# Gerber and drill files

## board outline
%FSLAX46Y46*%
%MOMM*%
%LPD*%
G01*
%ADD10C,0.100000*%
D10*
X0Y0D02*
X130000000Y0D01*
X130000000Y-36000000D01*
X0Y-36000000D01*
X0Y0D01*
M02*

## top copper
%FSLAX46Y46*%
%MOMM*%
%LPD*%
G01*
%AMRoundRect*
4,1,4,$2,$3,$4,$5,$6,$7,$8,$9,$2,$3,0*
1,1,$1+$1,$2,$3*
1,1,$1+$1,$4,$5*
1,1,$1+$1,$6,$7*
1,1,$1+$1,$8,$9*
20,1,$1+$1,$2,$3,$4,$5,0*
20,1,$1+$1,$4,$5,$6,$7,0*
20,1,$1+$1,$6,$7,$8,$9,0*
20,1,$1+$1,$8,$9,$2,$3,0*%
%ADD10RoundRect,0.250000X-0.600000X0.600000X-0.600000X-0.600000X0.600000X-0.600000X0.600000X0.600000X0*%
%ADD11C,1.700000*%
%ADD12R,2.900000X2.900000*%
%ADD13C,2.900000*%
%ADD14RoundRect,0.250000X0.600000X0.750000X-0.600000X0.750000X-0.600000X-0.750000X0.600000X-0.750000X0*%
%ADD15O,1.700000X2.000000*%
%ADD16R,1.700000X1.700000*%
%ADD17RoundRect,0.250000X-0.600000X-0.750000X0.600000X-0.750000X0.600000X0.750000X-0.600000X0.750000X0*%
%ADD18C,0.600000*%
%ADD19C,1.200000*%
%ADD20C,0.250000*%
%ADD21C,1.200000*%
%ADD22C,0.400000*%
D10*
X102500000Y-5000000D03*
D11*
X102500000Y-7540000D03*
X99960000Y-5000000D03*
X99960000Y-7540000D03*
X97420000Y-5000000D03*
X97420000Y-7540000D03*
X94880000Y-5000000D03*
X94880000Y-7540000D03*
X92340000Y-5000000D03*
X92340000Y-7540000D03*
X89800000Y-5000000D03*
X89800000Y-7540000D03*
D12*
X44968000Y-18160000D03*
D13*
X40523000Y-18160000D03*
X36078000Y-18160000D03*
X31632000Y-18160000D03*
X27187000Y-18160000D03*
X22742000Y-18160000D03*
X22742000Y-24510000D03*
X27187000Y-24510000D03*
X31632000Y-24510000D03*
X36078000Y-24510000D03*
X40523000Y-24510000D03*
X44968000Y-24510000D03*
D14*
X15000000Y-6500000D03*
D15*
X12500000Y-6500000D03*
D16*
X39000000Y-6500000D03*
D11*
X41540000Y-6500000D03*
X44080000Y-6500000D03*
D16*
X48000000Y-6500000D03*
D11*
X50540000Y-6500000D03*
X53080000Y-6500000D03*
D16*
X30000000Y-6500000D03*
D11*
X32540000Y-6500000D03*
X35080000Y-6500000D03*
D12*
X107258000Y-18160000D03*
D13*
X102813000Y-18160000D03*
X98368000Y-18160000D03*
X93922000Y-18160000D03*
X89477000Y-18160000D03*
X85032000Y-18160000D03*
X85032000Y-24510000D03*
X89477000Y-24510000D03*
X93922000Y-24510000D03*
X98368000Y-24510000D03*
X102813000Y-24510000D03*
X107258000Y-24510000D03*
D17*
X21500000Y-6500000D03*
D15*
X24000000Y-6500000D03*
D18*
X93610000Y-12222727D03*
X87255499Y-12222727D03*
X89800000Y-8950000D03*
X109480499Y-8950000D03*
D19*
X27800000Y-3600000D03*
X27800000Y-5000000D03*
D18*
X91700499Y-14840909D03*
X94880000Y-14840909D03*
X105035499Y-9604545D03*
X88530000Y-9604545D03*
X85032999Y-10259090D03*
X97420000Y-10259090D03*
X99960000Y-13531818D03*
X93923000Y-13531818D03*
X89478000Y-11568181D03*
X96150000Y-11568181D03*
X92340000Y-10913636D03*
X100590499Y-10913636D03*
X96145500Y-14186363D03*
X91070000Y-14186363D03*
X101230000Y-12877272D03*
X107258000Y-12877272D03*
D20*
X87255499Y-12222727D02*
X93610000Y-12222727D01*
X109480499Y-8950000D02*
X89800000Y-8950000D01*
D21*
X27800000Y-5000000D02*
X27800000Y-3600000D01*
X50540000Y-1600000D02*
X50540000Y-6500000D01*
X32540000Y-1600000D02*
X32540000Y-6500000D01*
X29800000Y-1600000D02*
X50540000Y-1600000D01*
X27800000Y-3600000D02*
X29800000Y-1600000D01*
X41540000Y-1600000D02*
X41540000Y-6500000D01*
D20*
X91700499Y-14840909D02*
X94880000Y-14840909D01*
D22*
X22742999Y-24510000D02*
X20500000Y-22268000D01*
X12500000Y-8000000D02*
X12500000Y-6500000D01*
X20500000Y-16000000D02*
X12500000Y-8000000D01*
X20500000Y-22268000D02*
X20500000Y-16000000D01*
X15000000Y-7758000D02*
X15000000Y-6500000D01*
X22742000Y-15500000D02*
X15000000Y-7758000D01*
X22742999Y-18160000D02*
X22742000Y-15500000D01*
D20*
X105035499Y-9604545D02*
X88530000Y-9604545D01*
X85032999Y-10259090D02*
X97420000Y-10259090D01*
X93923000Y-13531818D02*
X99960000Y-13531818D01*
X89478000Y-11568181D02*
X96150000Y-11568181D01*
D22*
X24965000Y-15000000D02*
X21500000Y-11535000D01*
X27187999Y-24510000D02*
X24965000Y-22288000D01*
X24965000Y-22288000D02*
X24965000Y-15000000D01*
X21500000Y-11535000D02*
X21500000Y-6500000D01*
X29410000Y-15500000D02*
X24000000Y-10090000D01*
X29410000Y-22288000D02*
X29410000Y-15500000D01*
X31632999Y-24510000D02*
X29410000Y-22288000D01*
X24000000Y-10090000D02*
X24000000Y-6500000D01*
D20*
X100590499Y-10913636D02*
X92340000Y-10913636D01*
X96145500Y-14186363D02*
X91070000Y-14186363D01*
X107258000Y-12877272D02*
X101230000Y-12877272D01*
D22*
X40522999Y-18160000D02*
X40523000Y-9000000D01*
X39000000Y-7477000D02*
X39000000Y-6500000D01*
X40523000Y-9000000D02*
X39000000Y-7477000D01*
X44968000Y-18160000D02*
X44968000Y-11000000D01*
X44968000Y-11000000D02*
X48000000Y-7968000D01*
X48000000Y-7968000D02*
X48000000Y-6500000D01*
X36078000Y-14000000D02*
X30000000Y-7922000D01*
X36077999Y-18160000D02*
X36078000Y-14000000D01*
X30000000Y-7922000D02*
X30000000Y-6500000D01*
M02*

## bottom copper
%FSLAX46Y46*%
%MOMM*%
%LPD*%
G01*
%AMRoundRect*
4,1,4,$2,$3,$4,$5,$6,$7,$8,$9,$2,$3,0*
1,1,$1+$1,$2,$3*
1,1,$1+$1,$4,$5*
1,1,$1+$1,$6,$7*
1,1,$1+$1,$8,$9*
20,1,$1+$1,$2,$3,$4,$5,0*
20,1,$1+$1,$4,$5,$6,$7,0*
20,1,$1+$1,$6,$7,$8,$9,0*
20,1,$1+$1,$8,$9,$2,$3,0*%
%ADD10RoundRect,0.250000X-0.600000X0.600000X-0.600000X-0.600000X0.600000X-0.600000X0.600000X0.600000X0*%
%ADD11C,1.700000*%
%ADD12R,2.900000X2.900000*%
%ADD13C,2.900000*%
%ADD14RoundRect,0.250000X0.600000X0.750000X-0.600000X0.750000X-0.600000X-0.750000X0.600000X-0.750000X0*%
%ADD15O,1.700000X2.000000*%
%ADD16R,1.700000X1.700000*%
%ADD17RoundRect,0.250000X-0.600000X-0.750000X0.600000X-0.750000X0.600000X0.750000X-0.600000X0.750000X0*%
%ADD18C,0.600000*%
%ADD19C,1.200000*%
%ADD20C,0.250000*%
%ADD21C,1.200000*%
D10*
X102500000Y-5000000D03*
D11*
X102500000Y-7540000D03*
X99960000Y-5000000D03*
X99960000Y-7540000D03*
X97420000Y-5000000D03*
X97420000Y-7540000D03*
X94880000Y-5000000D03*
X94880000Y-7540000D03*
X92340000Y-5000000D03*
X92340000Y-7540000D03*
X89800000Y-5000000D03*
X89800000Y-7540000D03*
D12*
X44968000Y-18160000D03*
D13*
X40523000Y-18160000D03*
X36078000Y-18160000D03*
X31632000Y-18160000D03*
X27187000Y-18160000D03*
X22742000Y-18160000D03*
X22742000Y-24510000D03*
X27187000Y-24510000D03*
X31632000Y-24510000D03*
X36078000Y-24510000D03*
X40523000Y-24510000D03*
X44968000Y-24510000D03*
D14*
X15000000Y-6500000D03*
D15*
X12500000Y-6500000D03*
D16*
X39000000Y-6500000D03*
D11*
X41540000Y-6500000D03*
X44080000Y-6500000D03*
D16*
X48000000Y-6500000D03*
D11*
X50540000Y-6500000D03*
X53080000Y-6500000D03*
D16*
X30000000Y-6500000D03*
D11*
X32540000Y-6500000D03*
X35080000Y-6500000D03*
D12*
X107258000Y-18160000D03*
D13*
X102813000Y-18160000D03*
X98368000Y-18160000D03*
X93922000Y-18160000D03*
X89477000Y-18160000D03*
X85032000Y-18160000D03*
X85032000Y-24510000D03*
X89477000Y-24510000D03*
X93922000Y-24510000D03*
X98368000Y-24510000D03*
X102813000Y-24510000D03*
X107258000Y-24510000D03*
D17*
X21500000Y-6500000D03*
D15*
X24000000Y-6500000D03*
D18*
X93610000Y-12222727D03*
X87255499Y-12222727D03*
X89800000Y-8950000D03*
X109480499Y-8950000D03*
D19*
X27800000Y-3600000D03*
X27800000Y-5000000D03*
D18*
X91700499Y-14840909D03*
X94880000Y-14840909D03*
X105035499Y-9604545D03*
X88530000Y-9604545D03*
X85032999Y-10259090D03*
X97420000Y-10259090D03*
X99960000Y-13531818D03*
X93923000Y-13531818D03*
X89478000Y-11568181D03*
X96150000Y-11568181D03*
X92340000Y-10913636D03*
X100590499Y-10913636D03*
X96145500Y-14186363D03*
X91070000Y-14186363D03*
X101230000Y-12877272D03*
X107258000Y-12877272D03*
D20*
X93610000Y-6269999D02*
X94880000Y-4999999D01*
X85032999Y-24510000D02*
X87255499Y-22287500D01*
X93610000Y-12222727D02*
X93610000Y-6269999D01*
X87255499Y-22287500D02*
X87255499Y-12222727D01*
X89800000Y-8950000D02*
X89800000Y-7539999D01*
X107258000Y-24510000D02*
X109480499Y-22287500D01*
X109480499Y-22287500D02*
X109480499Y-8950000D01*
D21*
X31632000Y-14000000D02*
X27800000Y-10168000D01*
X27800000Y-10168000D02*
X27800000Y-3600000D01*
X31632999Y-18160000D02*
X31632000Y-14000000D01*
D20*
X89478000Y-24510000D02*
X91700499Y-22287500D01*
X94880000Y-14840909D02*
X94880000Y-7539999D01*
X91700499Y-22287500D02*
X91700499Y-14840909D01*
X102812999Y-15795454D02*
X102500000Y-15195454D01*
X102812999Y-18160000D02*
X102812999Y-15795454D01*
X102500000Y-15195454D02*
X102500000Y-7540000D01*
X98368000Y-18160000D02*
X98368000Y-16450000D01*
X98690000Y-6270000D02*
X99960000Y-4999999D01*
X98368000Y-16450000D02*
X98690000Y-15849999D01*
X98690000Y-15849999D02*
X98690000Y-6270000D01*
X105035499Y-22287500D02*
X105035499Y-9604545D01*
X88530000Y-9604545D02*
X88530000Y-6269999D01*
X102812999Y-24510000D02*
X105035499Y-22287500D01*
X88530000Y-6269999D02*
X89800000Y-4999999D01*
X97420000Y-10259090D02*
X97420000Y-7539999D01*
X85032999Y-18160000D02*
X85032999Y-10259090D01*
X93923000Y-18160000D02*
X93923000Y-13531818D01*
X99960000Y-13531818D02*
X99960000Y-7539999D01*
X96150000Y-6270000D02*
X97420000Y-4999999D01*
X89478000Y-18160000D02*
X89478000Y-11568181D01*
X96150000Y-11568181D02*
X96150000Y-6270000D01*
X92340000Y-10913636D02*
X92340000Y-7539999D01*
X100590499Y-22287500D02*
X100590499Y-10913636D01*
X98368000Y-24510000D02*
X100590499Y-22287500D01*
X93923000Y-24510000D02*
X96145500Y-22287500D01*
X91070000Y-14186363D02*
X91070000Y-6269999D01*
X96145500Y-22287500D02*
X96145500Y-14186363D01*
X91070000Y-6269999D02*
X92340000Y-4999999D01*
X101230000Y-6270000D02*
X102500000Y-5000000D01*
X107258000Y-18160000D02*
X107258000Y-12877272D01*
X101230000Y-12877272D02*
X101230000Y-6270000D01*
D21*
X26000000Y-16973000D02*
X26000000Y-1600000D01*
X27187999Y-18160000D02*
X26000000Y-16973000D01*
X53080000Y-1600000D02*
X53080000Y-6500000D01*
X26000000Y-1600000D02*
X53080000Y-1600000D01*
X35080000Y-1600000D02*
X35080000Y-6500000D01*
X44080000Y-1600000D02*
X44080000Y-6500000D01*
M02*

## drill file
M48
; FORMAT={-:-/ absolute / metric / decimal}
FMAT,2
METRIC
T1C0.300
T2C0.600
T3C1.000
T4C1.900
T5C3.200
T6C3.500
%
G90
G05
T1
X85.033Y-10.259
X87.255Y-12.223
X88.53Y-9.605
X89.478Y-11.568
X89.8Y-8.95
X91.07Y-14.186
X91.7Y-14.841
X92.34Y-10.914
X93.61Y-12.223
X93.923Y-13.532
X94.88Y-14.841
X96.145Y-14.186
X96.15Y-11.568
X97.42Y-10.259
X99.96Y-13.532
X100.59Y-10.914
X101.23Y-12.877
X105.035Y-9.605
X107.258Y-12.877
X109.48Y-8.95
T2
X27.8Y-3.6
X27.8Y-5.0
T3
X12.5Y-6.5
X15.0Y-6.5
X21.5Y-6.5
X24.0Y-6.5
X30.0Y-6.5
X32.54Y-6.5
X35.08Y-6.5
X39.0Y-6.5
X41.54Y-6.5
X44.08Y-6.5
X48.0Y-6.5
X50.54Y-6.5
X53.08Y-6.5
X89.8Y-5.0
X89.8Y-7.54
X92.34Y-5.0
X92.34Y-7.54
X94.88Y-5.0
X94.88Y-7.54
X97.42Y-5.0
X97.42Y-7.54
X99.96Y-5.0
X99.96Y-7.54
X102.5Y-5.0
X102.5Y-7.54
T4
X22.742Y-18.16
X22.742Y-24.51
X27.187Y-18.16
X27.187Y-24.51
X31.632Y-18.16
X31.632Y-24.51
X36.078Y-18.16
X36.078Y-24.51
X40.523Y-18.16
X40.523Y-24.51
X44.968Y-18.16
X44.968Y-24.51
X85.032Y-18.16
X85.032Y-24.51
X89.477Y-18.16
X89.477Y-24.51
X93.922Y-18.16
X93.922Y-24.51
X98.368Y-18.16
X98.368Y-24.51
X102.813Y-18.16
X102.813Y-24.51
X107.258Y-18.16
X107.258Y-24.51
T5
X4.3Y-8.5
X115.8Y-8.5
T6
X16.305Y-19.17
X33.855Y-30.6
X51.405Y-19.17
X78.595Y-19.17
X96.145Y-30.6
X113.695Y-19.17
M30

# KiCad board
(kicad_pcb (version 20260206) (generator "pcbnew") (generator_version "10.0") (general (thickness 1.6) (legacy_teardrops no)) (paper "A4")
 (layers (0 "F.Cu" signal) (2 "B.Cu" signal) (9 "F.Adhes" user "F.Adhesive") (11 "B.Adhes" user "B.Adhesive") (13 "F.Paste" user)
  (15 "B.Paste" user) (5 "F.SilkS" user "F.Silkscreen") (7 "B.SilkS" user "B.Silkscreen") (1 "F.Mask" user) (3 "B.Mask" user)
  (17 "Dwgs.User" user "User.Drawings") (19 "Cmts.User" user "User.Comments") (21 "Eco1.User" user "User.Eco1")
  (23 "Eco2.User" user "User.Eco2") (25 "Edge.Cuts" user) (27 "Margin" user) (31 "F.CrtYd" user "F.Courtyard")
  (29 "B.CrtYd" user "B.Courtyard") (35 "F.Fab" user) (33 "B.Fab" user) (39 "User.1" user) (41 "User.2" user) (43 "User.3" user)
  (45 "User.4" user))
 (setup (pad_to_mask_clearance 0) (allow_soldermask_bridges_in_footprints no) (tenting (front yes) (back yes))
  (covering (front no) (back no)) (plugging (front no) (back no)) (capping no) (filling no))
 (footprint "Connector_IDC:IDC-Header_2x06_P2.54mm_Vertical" (layer "F.Cu") (at 102.5 5 -90)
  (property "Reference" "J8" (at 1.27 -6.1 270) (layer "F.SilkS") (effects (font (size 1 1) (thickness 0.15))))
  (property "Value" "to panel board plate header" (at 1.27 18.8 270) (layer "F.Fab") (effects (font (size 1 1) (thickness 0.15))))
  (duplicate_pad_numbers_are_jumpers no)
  (pad "1" thru_hole roundrect (at 0 0 270) (size 1.7 1.7) (drill 1) (layers "*.Cu" "*.Mask") (remove_unused_layers no)
   (roundrect_rratio 0.147059) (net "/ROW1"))
  (pad "2" thru_hole circle (at 2.54 0 270) (size 1.7 1.7) (drill 1) (layers "*.Cu" "*.Mask") (remove_unused_layers no) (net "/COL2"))
  (pad "3" thru_hole circle (at 0 2.54 270) (size 1.7 1.7) (drill 1) (layers "*.Cu" "*.Mask") (remove_unused_layers no) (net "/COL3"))
  (pad "4" thru_hole circle (at 2.54 2.54 270) (size 1.7 1.7) (drill 1) (layers "*.Cu" "*.Mask") (remove_unused_layers no) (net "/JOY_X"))
  (pad "5" thru_hole circle (at 0 5.08 270) (size 1.7 1.7) (drill 1) (layers "*.Cu" "*.Mask") (remove_unused_layers no) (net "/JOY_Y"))
  (pad "6" thru_hole circle (at 2.54 5.08 270) (size 1.7 1.7) (drill 1) (layers "*.Cu" "*.Mask") (remove_unused_layers no)
   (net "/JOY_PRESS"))
  (pad "7" thru_hole circle (at 0 7.62 270) (size 1.7 1.7) (drill 1) (layers "*.Cu" "*.Mask") (remove_unused_layers no) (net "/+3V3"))
  (pad "8" thru_hole circle (at 2.54 7.62 270) (size 1.7 1.7) (drill 1) (layers "*.Cu" "*.Mask") (remove_unused_layers no) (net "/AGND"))
  (pad "9" thru_hole circle (at 0 10.16 270) (size 1.7 1.7) (drill 1) (layers "*.Cu" "*.Mask") (remove_unused_layers no) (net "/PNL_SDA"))
  (pad "10" thru_hole circle (at 2.54 10.16 270) (size 1.7 1.7) (drill 1) (layers "*.Cu" "*.Mask") (remove_unused_layers no)
   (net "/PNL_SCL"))
  (pad "11" thru_hole circle (at 0 12.7 270) (size 1.7 1.7) (drill 1) (layers "*.Cu" "*.Mask") (remove_unused_layers no) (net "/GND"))
  (pad "12" thru_hole circle (at 2.54 12.7 270) (size 1.7 1.7) (drill 1) (layers "*.Cu" "*.Mask") (remove_unused_layers no) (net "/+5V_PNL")))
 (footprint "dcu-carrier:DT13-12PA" (layer "F.Cu") (at 33.855 19.17)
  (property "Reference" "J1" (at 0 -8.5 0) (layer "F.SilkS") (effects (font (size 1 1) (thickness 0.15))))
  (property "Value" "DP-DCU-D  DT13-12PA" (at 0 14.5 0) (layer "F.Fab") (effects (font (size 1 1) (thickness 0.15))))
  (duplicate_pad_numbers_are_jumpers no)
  (pad "" np_thru_hole circle (at -17.55 0) (size 3.5 3.5) (drill 3.5) (layers "*.Cu" "*.Mask"))
  (pad "" np_thru_hole circle (at 0 11.43) (size 3.5 3.5) (drill 3.5) (layers "*.Cu" "*.Mask"))
  (pad "" np_thru_hole circle (at 17.55 0) (size 3.5 3.5) (drill 3.5) (layers "*.Cu" "*.Mask"))
  (pad "1" thru_hole rect (at 11.113 -1.01) (size 2.9 2.9) (drill 1.9) (layers "*.Cu" "*.Mask") (remove_unused_layers no) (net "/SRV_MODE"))
  (pad "2" thru_hole circle (at 6.668 -1.01) (size 2.9 2.9) (drill 1.9) (layers "*.Cu" "*.Mask") (remove_unused_layers no)
   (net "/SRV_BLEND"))
  (pad "3" thru_hole circle (at 2.223 -1.01) (size 2.9 2.9) (drill 1.9) (layers "*.Cu" "*.Mask") (remove_unused_layers no)
   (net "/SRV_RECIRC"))
  (pad "4" thru_hole circle (at -2.223 -1.01) (size 2.9 2.9) (drill 1.9) (layers "*.Cu" "*.Mask") (remove_unused_layers no)
   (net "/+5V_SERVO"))
  (pad "5" thru_hole circle (at -6.668 -1.01) (size 2.9 2.9) (drill 1.9) (layers "*.Cu" "*.Mask") (remove_unused_layers no)
   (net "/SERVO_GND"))
  (pad "6" thru_hole circle (at -11.113 -1.01) (size 2.9 2.9) (drill 1.9) (layers "*.Cu" "*.Mask") (remove_unused_layers no)
   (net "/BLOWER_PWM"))
  (pad "7" thru_hole circle (at -11.113 5.34) (size 2.9 2.9) (drill 1.9) (layers "*.Cu" "*.Mask") (remove_unused_layers no)
   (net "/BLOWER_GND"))
  (pad "8" thru_hole circle (at -6.668 5.34) (size 2.9 2.9) (drill 1.9) (layers "*.Cu" "*.Mask") (remove_unused_layers no)
   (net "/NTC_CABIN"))
  (pad "9" thru_hole circle (at -2.223 5.34) (size 2.9 2.9) (drill 1.9) (layers "*.Cu" "*.Mask") (remove_unused_layers no) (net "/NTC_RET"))
  (pad "10" thru_hole circle (at 2.223 5.34) (size 2.9 2.9) (drill 1.9) (layers "*.Cu" "*.Mask") (remove_unused_layers no)
   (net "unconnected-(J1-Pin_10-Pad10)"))
  (pad "11" thru_hole circle (at 6.668 5.34) (size 2.9 2.9) (drill 1.9) (layers "*.Cu" "*.Mask") (remove_unused_layers no)
   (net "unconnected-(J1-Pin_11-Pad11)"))
  (pad "12" thru_hole circle (at 11.113 5.34) (size 2.9 2.9) (drill 1.9) (layers "*.Cu" "*.Mask") (remove_unused_layers no)
   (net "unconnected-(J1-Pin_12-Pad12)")))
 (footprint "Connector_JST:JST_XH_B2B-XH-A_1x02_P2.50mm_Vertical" (layer "F.Cu") (at 15 6.5 180)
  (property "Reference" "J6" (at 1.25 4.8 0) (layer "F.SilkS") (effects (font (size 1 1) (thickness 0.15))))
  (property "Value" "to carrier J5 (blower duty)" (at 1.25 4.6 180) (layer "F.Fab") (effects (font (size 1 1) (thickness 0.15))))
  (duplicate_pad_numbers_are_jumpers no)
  (pad "1" thru_hole roundrect (at 0 0 180) (size 1.7 2) (drill 1) (layers "*.Cu" "*.Mask") (remove_unused_layers no)
   (roundrect_rratio 0.147059) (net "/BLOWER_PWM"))
  (pad "2" thru_hole oval (at 2.5 0 180) (size 1.7 2) (drill 1) (layers "*.Cu" "*.Mask") (remove_unused_layers no) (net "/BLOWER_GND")))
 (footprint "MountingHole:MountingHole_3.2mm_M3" (layer "F.Cu") (at 115.8 8.5)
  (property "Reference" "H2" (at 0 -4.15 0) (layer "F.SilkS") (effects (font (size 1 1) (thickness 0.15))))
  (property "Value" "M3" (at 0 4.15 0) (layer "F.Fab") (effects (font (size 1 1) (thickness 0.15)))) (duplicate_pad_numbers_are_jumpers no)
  (pad "" np_thru_hole circle (at 0 0) (size 3.2 3.2) (drill 3.2) (layers "*.Cu" "*.Mask")))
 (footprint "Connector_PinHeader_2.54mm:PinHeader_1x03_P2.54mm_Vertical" (layer "F.Cu") (at 39 6.5 90)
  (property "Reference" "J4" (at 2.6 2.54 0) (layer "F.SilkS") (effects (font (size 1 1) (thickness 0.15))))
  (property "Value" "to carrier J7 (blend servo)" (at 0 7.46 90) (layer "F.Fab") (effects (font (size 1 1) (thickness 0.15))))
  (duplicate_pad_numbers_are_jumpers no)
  (pad "1" thru_hole rect (at 0 0 90) (size 1.7 1.7) (drill 1) (layers "*.Cu" "*.Mask") (remove_unused_layers no) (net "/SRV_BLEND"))
  (pad "2" thru_hole circle (at 0 2.54 90) (size 1.7 1.7) (drill 1) (layers "*.Cu" "*.Mask") (remove_unused_layers no) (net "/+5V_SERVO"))
  (pad "3" thru_hole circle (at 0 5.08 90) (size 1.7 1.7) (drill 1) (layers "*.Cu" "*.Mask") (remove_unused_layers no) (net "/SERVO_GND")))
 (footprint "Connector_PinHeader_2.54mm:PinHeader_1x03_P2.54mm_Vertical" (layer "F.Cu") (at 48 6.5 90)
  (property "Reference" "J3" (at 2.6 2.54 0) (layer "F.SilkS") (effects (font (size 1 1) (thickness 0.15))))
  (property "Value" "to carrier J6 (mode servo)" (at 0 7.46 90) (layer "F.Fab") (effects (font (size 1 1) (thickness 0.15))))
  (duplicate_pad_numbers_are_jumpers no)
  (pad "1" thru_hole rect (at 0 0 90) (size 1.7 1.7) (drill 1) (layers "*.Cu" "*.Mask") (remove_unused_layers no) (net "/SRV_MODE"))
  (pad "2" thru_hole circle (at 0 2.54 90) (size 1.7 1.7) (drill 1) (layers "*.Cu" "*.Mask") (remove_unused_layers no) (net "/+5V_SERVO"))
  (pad "3" thru_hole circle (at 0 5.08 90) (size 1.7 1.7) (drill 1) (layers "*.Cu" "*.Mask") (remove_unused_layers no) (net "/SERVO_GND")))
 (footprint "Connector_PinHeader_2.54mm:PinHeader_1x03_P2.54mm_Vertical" (layer "F.Cu") (at 30 6.5 90)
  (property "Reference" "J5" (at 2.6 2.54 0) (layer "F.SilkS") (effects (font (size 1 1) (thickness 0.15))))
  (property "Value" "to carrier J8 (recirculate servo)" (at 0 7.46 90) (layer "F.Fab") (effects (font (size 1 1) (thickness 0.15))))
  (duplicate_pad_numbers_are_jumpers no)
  (pad "1" thru_hole rect (at 0 0 90) (size 1.7 1.7) (drill 1) (layers "*.Cu" "*.Mask") (remove_unused_layers no) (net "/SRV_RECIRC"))
  (pad "2" thru_hole circle (at 0 2.54 90) (size 1.7 1.7) (drill 1) (layers "*.Cu" "*.Mask") (remove_unused_layers no) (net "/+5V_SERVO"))
  (pad "3" thru_hole circle (at 0 5.08 90) (size 1.7 1.7) (drill 1) (layers "*.Cu" "*.Mask") (remove_unused_layers no) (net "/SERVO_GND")))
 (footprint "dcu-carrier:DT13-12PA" (layer "F.Cu") (at 96.145 19.17)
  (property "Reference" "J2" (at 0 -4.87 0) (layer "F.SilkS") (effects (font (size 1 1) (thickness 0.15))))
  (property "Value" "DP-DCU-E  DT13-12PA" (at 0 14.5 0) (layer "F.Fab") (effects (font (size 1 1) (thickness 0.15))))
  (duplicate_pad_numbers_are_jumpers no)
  (pad "" np_thru_hole circle (at -17.55 0) (size 3.5 3.5) (drill 3.5) (layers "*.Cu" "*.Mask"))
  (pad "" np_thru_hole circle (at 0 11.43) (size 3.5 3.5) (drill 3.5) (layers "*.Cu" "*.Mask"))
  (pad "" np_thru_hole circle (at 17.55 0) (size 3.5 3.5) (drill 3.5) (layers "*.Cu" "*.Mask"))
  (pad "1" thru_hole rect (at 11.113 -1.01) (size 2.9 2.9) (drill 1.9) (layers "*.Cu" "*.Mask") (remove_unused_layers no) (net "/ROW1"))
  (pad "2" thru_hole circle (at 6.668 -1.01) (size 2.9 2.9) (drill 1.9) (layers "*.Cu" "*.Mask") (remove_unused_layers no) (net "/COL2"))
  (pad "3" thru_hole circle (at 2.223 -1.01) (size 2.9 2.9) (drill 1.9) (layers "*.Cu" "*.Mask") (remove_unused_layers no) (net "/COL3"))
  (pad "4" thru_hole circle (at -2.223 -1.01) (size 2.9 2.9) (drill 1.9) (layers "*.Cu" "*.Mask") (remove_unused_layers no) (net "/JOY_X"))
  (pad "5" thru_hole circle (at -6.668 -1.01) (size 2.9 2.9) (drill 1.9) (layers "*.Cu" "*.Mask") (remove_unused_layers no) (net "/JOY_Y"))
  (pad "6" thru_hole circle (at -11.113 -1.01) (size 2.9 2.9) (drill 1.9) (layers "*.Cu" "*.Mask") (remove_unused_layers no)
   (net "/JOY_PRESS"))
  (pad "7" thru_hole circle (at -11.113 5.34) (size 2.9 2.9) (drill 1.9) (layers "*.Cu" "*.Mask") (remove_unused_layers no) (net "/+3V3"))
  (pad "8" thru_hole circle (at -6.668 5.34) (size 2.9 2.9) (drill 1.9) (layers "*.Cu" "*.Mask") (remove_unused_layers no) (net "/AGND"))
  (pad "9" thru_hole circle (at -2.223 5.34) (size 2.9 2.9) (drill 1.9) (layers "*.Cu" "*.Mask") (remove_unused_layers no) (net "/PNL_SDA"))
  (pad "10" thru_hole circle (at 2.223 5.34) (size 2.9 2.9) (drill 1.9) (layers "*.Cu" "*.Mask") (remove_unused_layers no) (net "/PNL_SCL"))
  (pad "11" thru_hole circle (at 6.668 5.34) (size 2.9 2.9) (drill 1.9) (layers "*.Cu" "*.Mask") (remove_unused_layers no) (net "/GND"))
  (pad "12" thru_hole circle (at 11.113 5.34) (size 2.9 2.9) (drill 1.9) (layers "*.Cu" "*.Mask") (remove_unused_layers no) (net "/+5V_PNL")))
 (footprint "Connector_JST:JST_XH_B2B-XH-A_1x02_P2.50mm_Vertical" (layer "F.Cu") (at 21.5 6.5)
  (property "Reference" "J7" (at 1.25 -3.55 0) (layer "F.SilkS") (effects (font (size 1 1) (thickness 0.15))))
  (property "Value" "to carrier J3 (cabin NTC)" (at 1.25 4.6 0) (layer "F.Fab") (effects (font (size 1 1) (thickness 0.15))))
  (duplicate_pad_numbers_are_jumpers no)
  (pad "1" thru_hole roundrect (at 0 0) (size 1.7 2) (drill 1) (layers "*.Cu" "*.Mask") (remove_unused_layers no)
   (roundrect_rratio 0.147059) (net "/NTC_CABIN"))
  (pad "2" thru_hole oval (at 2.5 0) (size 1.7 2) (drill 1) (layers "*.Cu" "*.Mask") (remove_unused_layers no) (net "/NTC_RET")))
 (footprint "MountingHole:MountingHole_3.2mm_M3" (layer "F.Cu") (at 4.3 8.5)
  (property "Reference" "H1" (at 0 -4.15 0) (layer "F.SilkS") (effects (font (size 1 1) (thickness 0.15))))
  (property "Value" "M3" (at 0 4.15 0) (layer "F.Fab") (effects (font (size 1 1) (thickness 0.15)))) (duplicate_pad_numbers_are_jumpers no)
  (pad "" np_thru_hole circle (at 0 0) (size 3.2 3.2) (drill 3.2) (layers "*.Cu" "*.Mask")))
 (gr_rect (start 0 0) (end 130 36) (stroke (width 0.1) (type default)) (fill no) (layer "Edge.Cuts"))
 (segment (start 87.255499 12.222727) (end 93.61 12.222727) (width 0.25) (layer "F.Cu") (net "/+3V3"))
 (via (at 93.61 12.222727) (size 0.6) (drill 0.3) (layers "F.Cu" "B.Cu") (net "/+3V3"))
 (via (at 87.255499 12.222727) (size 0.6) (drill 0.3) (layers "F.Cu" "B.Cu") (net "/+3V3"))
 (segment (start 93.61 6.269999) (end 94.88 4.999999) (width 0.25) (layer "B.Cu") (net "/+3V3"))
 (segment (start 85.032999 24.51) (end 87.255499 22.2875) (width 0.25) (layer "B.Cu") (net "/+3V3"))
 (segment (start 93.61 12.222727) (end 93.61 6.269999) (width 0.25) (layer "B.Cu") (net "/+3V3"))
 (segment (start 87.255499 22.2875) (end 87.255499 12.222727) (width 0.25) (layer "B.Cu") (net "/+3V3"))
 (segment (start 109.480499 8.95) (end 89.8 8.95) (width 0.25) (layer "F.Cu") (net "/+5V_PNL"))
 (via (at 89.8 8.95) (size 0.6) (drill 0.3) (layers "F.Cu" "B.Cu") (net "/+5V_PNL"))
 (via (at 109.480499 8.95) (size 0.6) (drill 0.3) (layers "F.Cu" "B.Cu") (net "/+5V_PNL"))
 (segment (start 89.8 8.95) (end 89.8 7.539999) (width 0.25) (layer "B.Cu") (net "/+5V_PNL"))
 (segment (start 107.258 24.51) (end 109.480499 22.2875) (width 0.25) (layer "B.Cu") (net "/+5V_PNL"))
 (segment (start 109.480499 22.2875) (end 109.480499 8.95) (width 0.25) (layer "B.Cu") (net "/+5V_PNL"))
 (segment (start 27.8 5) (end 27.8 3.6) (width 1.2) (layer "F.Cu") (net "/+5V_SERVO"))
 (segment (start 50.54 1.6) (end 50.54 6.5) (width 1.2) (layer "F.Cu") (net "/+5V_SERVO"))
 (segment (start 32.54 1.6) (end 32.54 6.5) (width 1.2) (layer "F.Cu") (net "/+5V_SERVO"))
 (segment (start 29.8 1.6) (end 50.54 1.6) (width 1.2) (layer "F.Cu") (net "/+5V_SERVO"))
 (segment (start 27.8 3.6) (end 29.8 1.6) (width 1.2) (layer "F.Cu") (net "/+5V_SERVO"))
 (segment (start 41.54 1.6) (end 41.54 6.5) (width 1.2) (layer "F.Cu") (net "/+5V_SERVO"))
 (via (at 27.8 3.6) (size 1.2) (drill 0.6) (layers "F.Cu" "B.Cu") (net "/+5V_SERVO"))
 (via (at 27.8 5) (size 1.2) (drill 0.6) (layers "F.Cu" "B.Cu") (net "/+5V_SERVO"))
 (segment (start 31.632 14) (end 27.8 10.168) (width 1.2) (layer "B.Cu") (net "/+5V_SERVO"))
 (segment (start 27.8 10.168) (end 27.8 3.6) (width 1.2) (layer "B.Cu") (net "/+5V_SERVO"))
 (segment (start 31.632999 18.16) (end 31.632 14) (width 1.2) (layer "B.Cu") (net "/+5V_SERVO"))
 (segment (start 91.700499 14.840909) (end 94.88 14.840909) (width 0.25) (layer "F.Cu") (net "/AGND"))
 (via (at 91.700499 14.840909) (size 0.6) (drill 0.3) (layers "F.Cu" "B.Cu") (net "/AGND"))
 (via (at 94.88 14.840909) (size 0.6) (drill 0.3) (layers "F.Cu" "B.Cu") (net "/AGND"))
 (segment (start 89.478 24.51) (end 91.700499 22.2875) (width 0.25) (layer "B.Cu") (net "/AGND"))
 (segment (start 94.88 14.840909) (end 94.88 7.539999) (width 0.25) (layer "B.Cu") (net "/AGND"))
 (segment (start 91.700499 22.2875) (end 91.700499 14.840909) (width 0.25) (layer "B.Cu") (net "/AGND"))
 (segment (start 22.742999 24.51) (end 20.5 22.268) (width 0.4) (layer "F.Cu") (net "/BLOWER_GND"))
 (segment (start 12.5 8) (end 12.5 6.5) (width 0.4) (layer "F.Cu") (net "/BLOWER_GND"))
 (segment (start 20.5 16) (end 12.5 8) (width 0.4) (layer "F.Cu") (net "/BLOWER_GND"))
 (segment (start 20.5 22.268) (end 20.5 16) (width 0.4) (layer "F.Cu") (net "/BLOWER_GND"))
 (segment (start 15 7.758) (end 15 6.5) (width 0.4) (layer "F.Cu") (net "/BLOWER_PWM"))
 (segment (start 22.742 15.5) (end 15 7.758) (width 0.4) (layer "F.Cu") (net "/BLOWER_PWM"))
 (segment (start 22.742999 18.16) (end 22.742 15.5) (width 0.4) (layer "F.Cu") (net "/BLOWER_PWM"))
 (segment (start 102.812999 15.795454) (end 102.5 15.195454) (width 0.25) (layer "B.Cu") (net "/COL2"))
 (segment (start 102.812999 18.16) (end 102.812999 15.795454) (width 0.25) (layer "B.Cu") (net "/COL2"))
 (segment (start 102.5 15.195454) (end 102.5 7.54) (width 0.25) (layer "B.Cu") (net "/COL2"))
 (segment (start 98.368 18.16) (end 98.368 16.45) (width 0.25) (layer "B.Cu") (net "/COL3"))
 (segment (start 98.69 6.27) (end 99.96 4.999999) (width 0.25) (layer "B.Cu") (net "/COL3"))
 (segment (start 98.368 16.45) (end 98.69 15.849999) (width 0.25) (layer "B.Cu") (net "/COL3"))
 (segment (start 98.69 15.849999) (end 98.69 6.27) (width 0.25) (layer "B.Cu") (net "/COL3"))
 (segment (start 105.035499 9.604545) (end 88.53 9.604545) (width 0.25) (layer "F.Cu") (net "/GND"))
 (via (at 105.035499 9.604545) (size 0.6) (drill 0.3) (layers "F.Cu" "B.Cu") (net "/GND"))
 (via (at 88.53 9.604545) (size 0.6) (drill 0.3) (layers "F.Cu" "B.Cu") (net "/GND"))
 (segment (start 105.035499 22.2875) (end 105.035499 9.604545) (width 0.25) (layer "B.Cu") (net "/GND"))
 (segment (start 88.53 9.604545) (end 88.53 6.269999) (width 0.25) (layer "B.Cu") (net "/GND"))
 (segment (start 102.812999 24.51) (end 105.035499 22.2875) (width 0.25) (layer "B.Cu") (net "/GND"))
 (segment (start 88.53 6.269999) (end 89.8 4.999999) (width 0.25) (layer "B.Cu") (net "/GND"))
 (segment (start 85.032999 10.25909) (end 97.42 10.25909) (width 0.25) (layer "F.Cu") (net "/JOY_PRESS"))
 (via (at 85.032999 10.25909) (size 0.6) (drill 0.3) (layers "F.Cu" "B.Cu") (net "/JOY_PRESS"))
 (via (at 97.42 10.25909) (size 0.6) (drill 0.3) (layers "F.Cu" "B.Cu") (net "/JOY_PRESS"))
 (segment (start 97.42 10.25909) (end 97.42 7.539999) (width 0.25) (layer "B.Cu") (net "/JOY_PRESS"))
 (segment (start 85.032999 18.16) (end 85.032999 10.25909) (width 0.25) (layer "B.Cu") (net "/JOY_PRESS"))
 (segment (start 93.923 13.531818) (end 99.96 13.531818) (width 0.25) (layer "F.Cu") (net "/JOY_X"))
 (via (at 99.96 13.531818) (size 0.6) (drill 0.3) (layers "F.Cu" "B.Cu") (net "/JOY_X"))
 (via (at 93.923 13.531818) (size 0.6) (drill 0.3) (layers "F.Cu" "B.Cu") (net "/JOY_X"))
 (segment (start 93.923 18.16) (end 93.923 13.531818) (width 0.25) (layer "B.Cu") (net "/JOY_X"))
 (segment (start 99.96 13.531818) (end 99.96 7.539999) (width 0.25) (layer "B.Cu") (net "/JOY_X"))
 (segment (start 89.478 11.568181) (end 96.15 11.568181) (width 0.25) (layer "F.Cu") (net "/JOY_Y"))
 (via (at 89.478 11.568181) (size 0.6) (drill 0.3) (layers "F.Cu" "B.Cu") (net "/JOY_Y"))
 (via (at 96.15 11.568181) (size 0.6) (drill 0.3) (layers "F.Cu" "B.Cu") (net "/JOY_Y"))
 (segment (start 96.15 6.27) (end 97.42 4.999999) (width 0.25) (layer "B.Cu") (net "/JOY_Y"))
 (segment (start 89.478 18.16) (end 89.478 11.568181) (width 0.25) (layer "B.Cu") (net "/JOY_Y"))
 (segment (start 96.15 11.568181) (end 96.15 6.27) (width 0.25) (layer "B.Cu") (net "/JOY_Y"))
 (segment (start 24.965 15) (end 21.5 11.535) (width 0.4) (layer "F.Cu") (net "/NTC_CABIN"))
 (segment (start 27.187999 24.51) (end 24.965 22.288) (width 0.4) (layer "F.Cu") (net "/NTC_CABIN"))
 (segment (start 24.965 22.288) (end 24.965 15) (width 0.4) (layer "F.Cu") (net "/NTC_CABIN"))
 (segment (start 21.5 11.535) (end 21.5 6.5) (width 0.4) (layer "F.Cu") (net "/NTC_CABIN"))
 (segment (start 29.41 15.5) (end 24 10.09) (width 0.4) (layer "F.Cu") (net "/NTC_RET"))
 (segment (start 29.41 22.288) (end 29.41 15.5) (width 0.4) (layer "F.Cu") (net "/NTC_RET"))
 (segment (start 31.632999 24.51) (end 29.41 22.288) (width 0.4) (layer "F.Cu") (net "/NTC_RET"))
 (segment (start 24 10.09) (end 24 6.5) (width 0.4) (layer "F.Cu") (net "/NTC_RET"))
 (segment (start 100.590499 10.913636) (end 92.34 10.913636) (width 0.25) (layer "F.Cu") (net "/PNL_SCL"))
 (via (at 92.34 10.913636) (size 0.6) (drill 0.3) (layers "F.Cu" "B.Cu") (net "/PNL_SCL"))
 (via (at 100.590499 10.913636) (size 0.6) (drill 0.3) (layers "F.Cu" "B.Cu") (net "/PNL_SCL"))
 (segment (start 92.34 10.913636) (end 92.34 7.539999) (width 0.25) (layer "B.Cu") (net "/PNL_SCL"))
 (segment (start 100.590499 22.2875) (end 100.590499 10.913636) (width 0.25) (layer "B.Cu") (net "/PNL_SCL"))
 (segment (start 98.368 24.51) (end 100.590499 22.2875) (width 0.25) (layer "B.Cu") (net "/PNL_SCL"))
 (segment (start 96.1455 14.186363) (end 91.07 14.186363) (width 0.25) (layer "F.Cu") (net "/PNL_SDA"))
 (via (at 96.1455 14.186363) (size 0.6) (drill 0.3) (layers "F.Cu" "B.Cu") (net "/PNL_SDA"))
 (via (at 91.07 14.186363) (size 0.6) (drill 0.3) (layers "F.Cu" "B.Cu") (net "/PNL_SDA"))
 (segment (start 93.923 24.51) (end 96.1455 22.2875) (width 0.25) (layer "B.Cu") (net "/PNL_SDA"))
 (segment (start 91.07 14.186363) (end 91.07 6.269999) (width 0.25) (layer "B.Cu") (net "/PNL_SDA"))
 (segment (start 96.1455 22.2875) (end 96.1455 14.186363) (width 0.25) (layer "B.Cu") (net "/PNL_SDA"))
 (segment (start 91.07 6.269999) (end 92.34 4.999999) (width 0.25) (layer "B.Cu") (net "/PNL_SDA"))
 (segment (start 107.258 12.877272) (end 101.23 12.877272) (width 0.25) (layer "F.Cu") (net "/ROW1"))
 (via (at 101.23 12.877272) (size 0.6) (drill 0.3) (layers "F.Cu" "B.Cu") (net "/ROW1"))
 (via (at 107.258 12.877272) (size 0.6) (drill 0.3) (layers "F.Cu" "B.Cu") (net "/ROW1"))
 (segment (start 101.23 6.27) (end 102.5 5) (width 0.25) (layer "B.Cu") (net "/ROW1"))
 (segment (start 107.258 18.16) (end 107.258 12.877272) (width 0.25) (layer "B.Cu") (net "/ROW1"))
 (segment (start 101.23 12.877272) (end 101.23 6.27) (width 0.25) (layer "B.Cu") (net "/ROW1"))
 (segment (start 26 16.973) (end 26 1.6) (width 1.2) (layer "B.Cu") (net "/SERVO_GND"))
 (segment (start 27.187999 18.16) (end 26 16.973) (width 1.2) (layer "B.Cu") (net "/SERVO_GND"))
 (segment (start 53.08 1.6) (end 53.08 6.5) (width 1.2) (layer "B.Cu") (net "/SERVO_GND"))
 (segment (start 26 1.6) (end 53.08 1.6) (width 1.2) (layer "B.Cu") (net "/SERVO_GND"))
 (segment (start 35.08 1.6) (end 35.08 6.5) (width 1.2) (layer "B.Cu") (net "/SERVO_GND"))
 (segment (start 44.08 1.6) (end 44.08 6.5) (width 1.2) (layer "B.Cu") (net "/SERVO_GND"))
 (segment (start 40.522999 18.16) (end 40.523 9) (width 0.4) (layer "F.Cu") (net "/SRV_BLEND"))
 (segment (start 39 7.477) (end 39 6.5) (width 0.4) (layer "F.Cu") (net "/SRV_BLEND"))
 (segment (start 40.523 9) (end 39 7.477) (width 0.4) (layer "F.Cu") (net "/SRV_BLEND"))
 (segment (start 44.968 18.16) (end 44.968 11) (width 0.4) (layer "F.Cu") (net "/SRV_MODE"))
 (segment (start 44.968 11) (end 48 7.968) (width 0.4) (layer "F.Cu") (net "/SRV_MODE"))
 (segment (start 48 7.968) (end 48 6.5) (width 0.4) (layer "F.Cu") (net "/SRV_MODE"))
 (segment (start 36.078 14) (end 30 7.922) (width 0.4) (layer "F.Cu") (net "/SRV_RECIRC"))
 (segment (start 36.077999 18.16) (end 36.078 14) (width 0.4) (layer "F.Cu") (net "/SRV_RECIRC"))
 (segment (start 30 7.922) (end 30 6.5) (width 0.4) (layer "F.Cu") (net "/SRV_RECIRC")))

